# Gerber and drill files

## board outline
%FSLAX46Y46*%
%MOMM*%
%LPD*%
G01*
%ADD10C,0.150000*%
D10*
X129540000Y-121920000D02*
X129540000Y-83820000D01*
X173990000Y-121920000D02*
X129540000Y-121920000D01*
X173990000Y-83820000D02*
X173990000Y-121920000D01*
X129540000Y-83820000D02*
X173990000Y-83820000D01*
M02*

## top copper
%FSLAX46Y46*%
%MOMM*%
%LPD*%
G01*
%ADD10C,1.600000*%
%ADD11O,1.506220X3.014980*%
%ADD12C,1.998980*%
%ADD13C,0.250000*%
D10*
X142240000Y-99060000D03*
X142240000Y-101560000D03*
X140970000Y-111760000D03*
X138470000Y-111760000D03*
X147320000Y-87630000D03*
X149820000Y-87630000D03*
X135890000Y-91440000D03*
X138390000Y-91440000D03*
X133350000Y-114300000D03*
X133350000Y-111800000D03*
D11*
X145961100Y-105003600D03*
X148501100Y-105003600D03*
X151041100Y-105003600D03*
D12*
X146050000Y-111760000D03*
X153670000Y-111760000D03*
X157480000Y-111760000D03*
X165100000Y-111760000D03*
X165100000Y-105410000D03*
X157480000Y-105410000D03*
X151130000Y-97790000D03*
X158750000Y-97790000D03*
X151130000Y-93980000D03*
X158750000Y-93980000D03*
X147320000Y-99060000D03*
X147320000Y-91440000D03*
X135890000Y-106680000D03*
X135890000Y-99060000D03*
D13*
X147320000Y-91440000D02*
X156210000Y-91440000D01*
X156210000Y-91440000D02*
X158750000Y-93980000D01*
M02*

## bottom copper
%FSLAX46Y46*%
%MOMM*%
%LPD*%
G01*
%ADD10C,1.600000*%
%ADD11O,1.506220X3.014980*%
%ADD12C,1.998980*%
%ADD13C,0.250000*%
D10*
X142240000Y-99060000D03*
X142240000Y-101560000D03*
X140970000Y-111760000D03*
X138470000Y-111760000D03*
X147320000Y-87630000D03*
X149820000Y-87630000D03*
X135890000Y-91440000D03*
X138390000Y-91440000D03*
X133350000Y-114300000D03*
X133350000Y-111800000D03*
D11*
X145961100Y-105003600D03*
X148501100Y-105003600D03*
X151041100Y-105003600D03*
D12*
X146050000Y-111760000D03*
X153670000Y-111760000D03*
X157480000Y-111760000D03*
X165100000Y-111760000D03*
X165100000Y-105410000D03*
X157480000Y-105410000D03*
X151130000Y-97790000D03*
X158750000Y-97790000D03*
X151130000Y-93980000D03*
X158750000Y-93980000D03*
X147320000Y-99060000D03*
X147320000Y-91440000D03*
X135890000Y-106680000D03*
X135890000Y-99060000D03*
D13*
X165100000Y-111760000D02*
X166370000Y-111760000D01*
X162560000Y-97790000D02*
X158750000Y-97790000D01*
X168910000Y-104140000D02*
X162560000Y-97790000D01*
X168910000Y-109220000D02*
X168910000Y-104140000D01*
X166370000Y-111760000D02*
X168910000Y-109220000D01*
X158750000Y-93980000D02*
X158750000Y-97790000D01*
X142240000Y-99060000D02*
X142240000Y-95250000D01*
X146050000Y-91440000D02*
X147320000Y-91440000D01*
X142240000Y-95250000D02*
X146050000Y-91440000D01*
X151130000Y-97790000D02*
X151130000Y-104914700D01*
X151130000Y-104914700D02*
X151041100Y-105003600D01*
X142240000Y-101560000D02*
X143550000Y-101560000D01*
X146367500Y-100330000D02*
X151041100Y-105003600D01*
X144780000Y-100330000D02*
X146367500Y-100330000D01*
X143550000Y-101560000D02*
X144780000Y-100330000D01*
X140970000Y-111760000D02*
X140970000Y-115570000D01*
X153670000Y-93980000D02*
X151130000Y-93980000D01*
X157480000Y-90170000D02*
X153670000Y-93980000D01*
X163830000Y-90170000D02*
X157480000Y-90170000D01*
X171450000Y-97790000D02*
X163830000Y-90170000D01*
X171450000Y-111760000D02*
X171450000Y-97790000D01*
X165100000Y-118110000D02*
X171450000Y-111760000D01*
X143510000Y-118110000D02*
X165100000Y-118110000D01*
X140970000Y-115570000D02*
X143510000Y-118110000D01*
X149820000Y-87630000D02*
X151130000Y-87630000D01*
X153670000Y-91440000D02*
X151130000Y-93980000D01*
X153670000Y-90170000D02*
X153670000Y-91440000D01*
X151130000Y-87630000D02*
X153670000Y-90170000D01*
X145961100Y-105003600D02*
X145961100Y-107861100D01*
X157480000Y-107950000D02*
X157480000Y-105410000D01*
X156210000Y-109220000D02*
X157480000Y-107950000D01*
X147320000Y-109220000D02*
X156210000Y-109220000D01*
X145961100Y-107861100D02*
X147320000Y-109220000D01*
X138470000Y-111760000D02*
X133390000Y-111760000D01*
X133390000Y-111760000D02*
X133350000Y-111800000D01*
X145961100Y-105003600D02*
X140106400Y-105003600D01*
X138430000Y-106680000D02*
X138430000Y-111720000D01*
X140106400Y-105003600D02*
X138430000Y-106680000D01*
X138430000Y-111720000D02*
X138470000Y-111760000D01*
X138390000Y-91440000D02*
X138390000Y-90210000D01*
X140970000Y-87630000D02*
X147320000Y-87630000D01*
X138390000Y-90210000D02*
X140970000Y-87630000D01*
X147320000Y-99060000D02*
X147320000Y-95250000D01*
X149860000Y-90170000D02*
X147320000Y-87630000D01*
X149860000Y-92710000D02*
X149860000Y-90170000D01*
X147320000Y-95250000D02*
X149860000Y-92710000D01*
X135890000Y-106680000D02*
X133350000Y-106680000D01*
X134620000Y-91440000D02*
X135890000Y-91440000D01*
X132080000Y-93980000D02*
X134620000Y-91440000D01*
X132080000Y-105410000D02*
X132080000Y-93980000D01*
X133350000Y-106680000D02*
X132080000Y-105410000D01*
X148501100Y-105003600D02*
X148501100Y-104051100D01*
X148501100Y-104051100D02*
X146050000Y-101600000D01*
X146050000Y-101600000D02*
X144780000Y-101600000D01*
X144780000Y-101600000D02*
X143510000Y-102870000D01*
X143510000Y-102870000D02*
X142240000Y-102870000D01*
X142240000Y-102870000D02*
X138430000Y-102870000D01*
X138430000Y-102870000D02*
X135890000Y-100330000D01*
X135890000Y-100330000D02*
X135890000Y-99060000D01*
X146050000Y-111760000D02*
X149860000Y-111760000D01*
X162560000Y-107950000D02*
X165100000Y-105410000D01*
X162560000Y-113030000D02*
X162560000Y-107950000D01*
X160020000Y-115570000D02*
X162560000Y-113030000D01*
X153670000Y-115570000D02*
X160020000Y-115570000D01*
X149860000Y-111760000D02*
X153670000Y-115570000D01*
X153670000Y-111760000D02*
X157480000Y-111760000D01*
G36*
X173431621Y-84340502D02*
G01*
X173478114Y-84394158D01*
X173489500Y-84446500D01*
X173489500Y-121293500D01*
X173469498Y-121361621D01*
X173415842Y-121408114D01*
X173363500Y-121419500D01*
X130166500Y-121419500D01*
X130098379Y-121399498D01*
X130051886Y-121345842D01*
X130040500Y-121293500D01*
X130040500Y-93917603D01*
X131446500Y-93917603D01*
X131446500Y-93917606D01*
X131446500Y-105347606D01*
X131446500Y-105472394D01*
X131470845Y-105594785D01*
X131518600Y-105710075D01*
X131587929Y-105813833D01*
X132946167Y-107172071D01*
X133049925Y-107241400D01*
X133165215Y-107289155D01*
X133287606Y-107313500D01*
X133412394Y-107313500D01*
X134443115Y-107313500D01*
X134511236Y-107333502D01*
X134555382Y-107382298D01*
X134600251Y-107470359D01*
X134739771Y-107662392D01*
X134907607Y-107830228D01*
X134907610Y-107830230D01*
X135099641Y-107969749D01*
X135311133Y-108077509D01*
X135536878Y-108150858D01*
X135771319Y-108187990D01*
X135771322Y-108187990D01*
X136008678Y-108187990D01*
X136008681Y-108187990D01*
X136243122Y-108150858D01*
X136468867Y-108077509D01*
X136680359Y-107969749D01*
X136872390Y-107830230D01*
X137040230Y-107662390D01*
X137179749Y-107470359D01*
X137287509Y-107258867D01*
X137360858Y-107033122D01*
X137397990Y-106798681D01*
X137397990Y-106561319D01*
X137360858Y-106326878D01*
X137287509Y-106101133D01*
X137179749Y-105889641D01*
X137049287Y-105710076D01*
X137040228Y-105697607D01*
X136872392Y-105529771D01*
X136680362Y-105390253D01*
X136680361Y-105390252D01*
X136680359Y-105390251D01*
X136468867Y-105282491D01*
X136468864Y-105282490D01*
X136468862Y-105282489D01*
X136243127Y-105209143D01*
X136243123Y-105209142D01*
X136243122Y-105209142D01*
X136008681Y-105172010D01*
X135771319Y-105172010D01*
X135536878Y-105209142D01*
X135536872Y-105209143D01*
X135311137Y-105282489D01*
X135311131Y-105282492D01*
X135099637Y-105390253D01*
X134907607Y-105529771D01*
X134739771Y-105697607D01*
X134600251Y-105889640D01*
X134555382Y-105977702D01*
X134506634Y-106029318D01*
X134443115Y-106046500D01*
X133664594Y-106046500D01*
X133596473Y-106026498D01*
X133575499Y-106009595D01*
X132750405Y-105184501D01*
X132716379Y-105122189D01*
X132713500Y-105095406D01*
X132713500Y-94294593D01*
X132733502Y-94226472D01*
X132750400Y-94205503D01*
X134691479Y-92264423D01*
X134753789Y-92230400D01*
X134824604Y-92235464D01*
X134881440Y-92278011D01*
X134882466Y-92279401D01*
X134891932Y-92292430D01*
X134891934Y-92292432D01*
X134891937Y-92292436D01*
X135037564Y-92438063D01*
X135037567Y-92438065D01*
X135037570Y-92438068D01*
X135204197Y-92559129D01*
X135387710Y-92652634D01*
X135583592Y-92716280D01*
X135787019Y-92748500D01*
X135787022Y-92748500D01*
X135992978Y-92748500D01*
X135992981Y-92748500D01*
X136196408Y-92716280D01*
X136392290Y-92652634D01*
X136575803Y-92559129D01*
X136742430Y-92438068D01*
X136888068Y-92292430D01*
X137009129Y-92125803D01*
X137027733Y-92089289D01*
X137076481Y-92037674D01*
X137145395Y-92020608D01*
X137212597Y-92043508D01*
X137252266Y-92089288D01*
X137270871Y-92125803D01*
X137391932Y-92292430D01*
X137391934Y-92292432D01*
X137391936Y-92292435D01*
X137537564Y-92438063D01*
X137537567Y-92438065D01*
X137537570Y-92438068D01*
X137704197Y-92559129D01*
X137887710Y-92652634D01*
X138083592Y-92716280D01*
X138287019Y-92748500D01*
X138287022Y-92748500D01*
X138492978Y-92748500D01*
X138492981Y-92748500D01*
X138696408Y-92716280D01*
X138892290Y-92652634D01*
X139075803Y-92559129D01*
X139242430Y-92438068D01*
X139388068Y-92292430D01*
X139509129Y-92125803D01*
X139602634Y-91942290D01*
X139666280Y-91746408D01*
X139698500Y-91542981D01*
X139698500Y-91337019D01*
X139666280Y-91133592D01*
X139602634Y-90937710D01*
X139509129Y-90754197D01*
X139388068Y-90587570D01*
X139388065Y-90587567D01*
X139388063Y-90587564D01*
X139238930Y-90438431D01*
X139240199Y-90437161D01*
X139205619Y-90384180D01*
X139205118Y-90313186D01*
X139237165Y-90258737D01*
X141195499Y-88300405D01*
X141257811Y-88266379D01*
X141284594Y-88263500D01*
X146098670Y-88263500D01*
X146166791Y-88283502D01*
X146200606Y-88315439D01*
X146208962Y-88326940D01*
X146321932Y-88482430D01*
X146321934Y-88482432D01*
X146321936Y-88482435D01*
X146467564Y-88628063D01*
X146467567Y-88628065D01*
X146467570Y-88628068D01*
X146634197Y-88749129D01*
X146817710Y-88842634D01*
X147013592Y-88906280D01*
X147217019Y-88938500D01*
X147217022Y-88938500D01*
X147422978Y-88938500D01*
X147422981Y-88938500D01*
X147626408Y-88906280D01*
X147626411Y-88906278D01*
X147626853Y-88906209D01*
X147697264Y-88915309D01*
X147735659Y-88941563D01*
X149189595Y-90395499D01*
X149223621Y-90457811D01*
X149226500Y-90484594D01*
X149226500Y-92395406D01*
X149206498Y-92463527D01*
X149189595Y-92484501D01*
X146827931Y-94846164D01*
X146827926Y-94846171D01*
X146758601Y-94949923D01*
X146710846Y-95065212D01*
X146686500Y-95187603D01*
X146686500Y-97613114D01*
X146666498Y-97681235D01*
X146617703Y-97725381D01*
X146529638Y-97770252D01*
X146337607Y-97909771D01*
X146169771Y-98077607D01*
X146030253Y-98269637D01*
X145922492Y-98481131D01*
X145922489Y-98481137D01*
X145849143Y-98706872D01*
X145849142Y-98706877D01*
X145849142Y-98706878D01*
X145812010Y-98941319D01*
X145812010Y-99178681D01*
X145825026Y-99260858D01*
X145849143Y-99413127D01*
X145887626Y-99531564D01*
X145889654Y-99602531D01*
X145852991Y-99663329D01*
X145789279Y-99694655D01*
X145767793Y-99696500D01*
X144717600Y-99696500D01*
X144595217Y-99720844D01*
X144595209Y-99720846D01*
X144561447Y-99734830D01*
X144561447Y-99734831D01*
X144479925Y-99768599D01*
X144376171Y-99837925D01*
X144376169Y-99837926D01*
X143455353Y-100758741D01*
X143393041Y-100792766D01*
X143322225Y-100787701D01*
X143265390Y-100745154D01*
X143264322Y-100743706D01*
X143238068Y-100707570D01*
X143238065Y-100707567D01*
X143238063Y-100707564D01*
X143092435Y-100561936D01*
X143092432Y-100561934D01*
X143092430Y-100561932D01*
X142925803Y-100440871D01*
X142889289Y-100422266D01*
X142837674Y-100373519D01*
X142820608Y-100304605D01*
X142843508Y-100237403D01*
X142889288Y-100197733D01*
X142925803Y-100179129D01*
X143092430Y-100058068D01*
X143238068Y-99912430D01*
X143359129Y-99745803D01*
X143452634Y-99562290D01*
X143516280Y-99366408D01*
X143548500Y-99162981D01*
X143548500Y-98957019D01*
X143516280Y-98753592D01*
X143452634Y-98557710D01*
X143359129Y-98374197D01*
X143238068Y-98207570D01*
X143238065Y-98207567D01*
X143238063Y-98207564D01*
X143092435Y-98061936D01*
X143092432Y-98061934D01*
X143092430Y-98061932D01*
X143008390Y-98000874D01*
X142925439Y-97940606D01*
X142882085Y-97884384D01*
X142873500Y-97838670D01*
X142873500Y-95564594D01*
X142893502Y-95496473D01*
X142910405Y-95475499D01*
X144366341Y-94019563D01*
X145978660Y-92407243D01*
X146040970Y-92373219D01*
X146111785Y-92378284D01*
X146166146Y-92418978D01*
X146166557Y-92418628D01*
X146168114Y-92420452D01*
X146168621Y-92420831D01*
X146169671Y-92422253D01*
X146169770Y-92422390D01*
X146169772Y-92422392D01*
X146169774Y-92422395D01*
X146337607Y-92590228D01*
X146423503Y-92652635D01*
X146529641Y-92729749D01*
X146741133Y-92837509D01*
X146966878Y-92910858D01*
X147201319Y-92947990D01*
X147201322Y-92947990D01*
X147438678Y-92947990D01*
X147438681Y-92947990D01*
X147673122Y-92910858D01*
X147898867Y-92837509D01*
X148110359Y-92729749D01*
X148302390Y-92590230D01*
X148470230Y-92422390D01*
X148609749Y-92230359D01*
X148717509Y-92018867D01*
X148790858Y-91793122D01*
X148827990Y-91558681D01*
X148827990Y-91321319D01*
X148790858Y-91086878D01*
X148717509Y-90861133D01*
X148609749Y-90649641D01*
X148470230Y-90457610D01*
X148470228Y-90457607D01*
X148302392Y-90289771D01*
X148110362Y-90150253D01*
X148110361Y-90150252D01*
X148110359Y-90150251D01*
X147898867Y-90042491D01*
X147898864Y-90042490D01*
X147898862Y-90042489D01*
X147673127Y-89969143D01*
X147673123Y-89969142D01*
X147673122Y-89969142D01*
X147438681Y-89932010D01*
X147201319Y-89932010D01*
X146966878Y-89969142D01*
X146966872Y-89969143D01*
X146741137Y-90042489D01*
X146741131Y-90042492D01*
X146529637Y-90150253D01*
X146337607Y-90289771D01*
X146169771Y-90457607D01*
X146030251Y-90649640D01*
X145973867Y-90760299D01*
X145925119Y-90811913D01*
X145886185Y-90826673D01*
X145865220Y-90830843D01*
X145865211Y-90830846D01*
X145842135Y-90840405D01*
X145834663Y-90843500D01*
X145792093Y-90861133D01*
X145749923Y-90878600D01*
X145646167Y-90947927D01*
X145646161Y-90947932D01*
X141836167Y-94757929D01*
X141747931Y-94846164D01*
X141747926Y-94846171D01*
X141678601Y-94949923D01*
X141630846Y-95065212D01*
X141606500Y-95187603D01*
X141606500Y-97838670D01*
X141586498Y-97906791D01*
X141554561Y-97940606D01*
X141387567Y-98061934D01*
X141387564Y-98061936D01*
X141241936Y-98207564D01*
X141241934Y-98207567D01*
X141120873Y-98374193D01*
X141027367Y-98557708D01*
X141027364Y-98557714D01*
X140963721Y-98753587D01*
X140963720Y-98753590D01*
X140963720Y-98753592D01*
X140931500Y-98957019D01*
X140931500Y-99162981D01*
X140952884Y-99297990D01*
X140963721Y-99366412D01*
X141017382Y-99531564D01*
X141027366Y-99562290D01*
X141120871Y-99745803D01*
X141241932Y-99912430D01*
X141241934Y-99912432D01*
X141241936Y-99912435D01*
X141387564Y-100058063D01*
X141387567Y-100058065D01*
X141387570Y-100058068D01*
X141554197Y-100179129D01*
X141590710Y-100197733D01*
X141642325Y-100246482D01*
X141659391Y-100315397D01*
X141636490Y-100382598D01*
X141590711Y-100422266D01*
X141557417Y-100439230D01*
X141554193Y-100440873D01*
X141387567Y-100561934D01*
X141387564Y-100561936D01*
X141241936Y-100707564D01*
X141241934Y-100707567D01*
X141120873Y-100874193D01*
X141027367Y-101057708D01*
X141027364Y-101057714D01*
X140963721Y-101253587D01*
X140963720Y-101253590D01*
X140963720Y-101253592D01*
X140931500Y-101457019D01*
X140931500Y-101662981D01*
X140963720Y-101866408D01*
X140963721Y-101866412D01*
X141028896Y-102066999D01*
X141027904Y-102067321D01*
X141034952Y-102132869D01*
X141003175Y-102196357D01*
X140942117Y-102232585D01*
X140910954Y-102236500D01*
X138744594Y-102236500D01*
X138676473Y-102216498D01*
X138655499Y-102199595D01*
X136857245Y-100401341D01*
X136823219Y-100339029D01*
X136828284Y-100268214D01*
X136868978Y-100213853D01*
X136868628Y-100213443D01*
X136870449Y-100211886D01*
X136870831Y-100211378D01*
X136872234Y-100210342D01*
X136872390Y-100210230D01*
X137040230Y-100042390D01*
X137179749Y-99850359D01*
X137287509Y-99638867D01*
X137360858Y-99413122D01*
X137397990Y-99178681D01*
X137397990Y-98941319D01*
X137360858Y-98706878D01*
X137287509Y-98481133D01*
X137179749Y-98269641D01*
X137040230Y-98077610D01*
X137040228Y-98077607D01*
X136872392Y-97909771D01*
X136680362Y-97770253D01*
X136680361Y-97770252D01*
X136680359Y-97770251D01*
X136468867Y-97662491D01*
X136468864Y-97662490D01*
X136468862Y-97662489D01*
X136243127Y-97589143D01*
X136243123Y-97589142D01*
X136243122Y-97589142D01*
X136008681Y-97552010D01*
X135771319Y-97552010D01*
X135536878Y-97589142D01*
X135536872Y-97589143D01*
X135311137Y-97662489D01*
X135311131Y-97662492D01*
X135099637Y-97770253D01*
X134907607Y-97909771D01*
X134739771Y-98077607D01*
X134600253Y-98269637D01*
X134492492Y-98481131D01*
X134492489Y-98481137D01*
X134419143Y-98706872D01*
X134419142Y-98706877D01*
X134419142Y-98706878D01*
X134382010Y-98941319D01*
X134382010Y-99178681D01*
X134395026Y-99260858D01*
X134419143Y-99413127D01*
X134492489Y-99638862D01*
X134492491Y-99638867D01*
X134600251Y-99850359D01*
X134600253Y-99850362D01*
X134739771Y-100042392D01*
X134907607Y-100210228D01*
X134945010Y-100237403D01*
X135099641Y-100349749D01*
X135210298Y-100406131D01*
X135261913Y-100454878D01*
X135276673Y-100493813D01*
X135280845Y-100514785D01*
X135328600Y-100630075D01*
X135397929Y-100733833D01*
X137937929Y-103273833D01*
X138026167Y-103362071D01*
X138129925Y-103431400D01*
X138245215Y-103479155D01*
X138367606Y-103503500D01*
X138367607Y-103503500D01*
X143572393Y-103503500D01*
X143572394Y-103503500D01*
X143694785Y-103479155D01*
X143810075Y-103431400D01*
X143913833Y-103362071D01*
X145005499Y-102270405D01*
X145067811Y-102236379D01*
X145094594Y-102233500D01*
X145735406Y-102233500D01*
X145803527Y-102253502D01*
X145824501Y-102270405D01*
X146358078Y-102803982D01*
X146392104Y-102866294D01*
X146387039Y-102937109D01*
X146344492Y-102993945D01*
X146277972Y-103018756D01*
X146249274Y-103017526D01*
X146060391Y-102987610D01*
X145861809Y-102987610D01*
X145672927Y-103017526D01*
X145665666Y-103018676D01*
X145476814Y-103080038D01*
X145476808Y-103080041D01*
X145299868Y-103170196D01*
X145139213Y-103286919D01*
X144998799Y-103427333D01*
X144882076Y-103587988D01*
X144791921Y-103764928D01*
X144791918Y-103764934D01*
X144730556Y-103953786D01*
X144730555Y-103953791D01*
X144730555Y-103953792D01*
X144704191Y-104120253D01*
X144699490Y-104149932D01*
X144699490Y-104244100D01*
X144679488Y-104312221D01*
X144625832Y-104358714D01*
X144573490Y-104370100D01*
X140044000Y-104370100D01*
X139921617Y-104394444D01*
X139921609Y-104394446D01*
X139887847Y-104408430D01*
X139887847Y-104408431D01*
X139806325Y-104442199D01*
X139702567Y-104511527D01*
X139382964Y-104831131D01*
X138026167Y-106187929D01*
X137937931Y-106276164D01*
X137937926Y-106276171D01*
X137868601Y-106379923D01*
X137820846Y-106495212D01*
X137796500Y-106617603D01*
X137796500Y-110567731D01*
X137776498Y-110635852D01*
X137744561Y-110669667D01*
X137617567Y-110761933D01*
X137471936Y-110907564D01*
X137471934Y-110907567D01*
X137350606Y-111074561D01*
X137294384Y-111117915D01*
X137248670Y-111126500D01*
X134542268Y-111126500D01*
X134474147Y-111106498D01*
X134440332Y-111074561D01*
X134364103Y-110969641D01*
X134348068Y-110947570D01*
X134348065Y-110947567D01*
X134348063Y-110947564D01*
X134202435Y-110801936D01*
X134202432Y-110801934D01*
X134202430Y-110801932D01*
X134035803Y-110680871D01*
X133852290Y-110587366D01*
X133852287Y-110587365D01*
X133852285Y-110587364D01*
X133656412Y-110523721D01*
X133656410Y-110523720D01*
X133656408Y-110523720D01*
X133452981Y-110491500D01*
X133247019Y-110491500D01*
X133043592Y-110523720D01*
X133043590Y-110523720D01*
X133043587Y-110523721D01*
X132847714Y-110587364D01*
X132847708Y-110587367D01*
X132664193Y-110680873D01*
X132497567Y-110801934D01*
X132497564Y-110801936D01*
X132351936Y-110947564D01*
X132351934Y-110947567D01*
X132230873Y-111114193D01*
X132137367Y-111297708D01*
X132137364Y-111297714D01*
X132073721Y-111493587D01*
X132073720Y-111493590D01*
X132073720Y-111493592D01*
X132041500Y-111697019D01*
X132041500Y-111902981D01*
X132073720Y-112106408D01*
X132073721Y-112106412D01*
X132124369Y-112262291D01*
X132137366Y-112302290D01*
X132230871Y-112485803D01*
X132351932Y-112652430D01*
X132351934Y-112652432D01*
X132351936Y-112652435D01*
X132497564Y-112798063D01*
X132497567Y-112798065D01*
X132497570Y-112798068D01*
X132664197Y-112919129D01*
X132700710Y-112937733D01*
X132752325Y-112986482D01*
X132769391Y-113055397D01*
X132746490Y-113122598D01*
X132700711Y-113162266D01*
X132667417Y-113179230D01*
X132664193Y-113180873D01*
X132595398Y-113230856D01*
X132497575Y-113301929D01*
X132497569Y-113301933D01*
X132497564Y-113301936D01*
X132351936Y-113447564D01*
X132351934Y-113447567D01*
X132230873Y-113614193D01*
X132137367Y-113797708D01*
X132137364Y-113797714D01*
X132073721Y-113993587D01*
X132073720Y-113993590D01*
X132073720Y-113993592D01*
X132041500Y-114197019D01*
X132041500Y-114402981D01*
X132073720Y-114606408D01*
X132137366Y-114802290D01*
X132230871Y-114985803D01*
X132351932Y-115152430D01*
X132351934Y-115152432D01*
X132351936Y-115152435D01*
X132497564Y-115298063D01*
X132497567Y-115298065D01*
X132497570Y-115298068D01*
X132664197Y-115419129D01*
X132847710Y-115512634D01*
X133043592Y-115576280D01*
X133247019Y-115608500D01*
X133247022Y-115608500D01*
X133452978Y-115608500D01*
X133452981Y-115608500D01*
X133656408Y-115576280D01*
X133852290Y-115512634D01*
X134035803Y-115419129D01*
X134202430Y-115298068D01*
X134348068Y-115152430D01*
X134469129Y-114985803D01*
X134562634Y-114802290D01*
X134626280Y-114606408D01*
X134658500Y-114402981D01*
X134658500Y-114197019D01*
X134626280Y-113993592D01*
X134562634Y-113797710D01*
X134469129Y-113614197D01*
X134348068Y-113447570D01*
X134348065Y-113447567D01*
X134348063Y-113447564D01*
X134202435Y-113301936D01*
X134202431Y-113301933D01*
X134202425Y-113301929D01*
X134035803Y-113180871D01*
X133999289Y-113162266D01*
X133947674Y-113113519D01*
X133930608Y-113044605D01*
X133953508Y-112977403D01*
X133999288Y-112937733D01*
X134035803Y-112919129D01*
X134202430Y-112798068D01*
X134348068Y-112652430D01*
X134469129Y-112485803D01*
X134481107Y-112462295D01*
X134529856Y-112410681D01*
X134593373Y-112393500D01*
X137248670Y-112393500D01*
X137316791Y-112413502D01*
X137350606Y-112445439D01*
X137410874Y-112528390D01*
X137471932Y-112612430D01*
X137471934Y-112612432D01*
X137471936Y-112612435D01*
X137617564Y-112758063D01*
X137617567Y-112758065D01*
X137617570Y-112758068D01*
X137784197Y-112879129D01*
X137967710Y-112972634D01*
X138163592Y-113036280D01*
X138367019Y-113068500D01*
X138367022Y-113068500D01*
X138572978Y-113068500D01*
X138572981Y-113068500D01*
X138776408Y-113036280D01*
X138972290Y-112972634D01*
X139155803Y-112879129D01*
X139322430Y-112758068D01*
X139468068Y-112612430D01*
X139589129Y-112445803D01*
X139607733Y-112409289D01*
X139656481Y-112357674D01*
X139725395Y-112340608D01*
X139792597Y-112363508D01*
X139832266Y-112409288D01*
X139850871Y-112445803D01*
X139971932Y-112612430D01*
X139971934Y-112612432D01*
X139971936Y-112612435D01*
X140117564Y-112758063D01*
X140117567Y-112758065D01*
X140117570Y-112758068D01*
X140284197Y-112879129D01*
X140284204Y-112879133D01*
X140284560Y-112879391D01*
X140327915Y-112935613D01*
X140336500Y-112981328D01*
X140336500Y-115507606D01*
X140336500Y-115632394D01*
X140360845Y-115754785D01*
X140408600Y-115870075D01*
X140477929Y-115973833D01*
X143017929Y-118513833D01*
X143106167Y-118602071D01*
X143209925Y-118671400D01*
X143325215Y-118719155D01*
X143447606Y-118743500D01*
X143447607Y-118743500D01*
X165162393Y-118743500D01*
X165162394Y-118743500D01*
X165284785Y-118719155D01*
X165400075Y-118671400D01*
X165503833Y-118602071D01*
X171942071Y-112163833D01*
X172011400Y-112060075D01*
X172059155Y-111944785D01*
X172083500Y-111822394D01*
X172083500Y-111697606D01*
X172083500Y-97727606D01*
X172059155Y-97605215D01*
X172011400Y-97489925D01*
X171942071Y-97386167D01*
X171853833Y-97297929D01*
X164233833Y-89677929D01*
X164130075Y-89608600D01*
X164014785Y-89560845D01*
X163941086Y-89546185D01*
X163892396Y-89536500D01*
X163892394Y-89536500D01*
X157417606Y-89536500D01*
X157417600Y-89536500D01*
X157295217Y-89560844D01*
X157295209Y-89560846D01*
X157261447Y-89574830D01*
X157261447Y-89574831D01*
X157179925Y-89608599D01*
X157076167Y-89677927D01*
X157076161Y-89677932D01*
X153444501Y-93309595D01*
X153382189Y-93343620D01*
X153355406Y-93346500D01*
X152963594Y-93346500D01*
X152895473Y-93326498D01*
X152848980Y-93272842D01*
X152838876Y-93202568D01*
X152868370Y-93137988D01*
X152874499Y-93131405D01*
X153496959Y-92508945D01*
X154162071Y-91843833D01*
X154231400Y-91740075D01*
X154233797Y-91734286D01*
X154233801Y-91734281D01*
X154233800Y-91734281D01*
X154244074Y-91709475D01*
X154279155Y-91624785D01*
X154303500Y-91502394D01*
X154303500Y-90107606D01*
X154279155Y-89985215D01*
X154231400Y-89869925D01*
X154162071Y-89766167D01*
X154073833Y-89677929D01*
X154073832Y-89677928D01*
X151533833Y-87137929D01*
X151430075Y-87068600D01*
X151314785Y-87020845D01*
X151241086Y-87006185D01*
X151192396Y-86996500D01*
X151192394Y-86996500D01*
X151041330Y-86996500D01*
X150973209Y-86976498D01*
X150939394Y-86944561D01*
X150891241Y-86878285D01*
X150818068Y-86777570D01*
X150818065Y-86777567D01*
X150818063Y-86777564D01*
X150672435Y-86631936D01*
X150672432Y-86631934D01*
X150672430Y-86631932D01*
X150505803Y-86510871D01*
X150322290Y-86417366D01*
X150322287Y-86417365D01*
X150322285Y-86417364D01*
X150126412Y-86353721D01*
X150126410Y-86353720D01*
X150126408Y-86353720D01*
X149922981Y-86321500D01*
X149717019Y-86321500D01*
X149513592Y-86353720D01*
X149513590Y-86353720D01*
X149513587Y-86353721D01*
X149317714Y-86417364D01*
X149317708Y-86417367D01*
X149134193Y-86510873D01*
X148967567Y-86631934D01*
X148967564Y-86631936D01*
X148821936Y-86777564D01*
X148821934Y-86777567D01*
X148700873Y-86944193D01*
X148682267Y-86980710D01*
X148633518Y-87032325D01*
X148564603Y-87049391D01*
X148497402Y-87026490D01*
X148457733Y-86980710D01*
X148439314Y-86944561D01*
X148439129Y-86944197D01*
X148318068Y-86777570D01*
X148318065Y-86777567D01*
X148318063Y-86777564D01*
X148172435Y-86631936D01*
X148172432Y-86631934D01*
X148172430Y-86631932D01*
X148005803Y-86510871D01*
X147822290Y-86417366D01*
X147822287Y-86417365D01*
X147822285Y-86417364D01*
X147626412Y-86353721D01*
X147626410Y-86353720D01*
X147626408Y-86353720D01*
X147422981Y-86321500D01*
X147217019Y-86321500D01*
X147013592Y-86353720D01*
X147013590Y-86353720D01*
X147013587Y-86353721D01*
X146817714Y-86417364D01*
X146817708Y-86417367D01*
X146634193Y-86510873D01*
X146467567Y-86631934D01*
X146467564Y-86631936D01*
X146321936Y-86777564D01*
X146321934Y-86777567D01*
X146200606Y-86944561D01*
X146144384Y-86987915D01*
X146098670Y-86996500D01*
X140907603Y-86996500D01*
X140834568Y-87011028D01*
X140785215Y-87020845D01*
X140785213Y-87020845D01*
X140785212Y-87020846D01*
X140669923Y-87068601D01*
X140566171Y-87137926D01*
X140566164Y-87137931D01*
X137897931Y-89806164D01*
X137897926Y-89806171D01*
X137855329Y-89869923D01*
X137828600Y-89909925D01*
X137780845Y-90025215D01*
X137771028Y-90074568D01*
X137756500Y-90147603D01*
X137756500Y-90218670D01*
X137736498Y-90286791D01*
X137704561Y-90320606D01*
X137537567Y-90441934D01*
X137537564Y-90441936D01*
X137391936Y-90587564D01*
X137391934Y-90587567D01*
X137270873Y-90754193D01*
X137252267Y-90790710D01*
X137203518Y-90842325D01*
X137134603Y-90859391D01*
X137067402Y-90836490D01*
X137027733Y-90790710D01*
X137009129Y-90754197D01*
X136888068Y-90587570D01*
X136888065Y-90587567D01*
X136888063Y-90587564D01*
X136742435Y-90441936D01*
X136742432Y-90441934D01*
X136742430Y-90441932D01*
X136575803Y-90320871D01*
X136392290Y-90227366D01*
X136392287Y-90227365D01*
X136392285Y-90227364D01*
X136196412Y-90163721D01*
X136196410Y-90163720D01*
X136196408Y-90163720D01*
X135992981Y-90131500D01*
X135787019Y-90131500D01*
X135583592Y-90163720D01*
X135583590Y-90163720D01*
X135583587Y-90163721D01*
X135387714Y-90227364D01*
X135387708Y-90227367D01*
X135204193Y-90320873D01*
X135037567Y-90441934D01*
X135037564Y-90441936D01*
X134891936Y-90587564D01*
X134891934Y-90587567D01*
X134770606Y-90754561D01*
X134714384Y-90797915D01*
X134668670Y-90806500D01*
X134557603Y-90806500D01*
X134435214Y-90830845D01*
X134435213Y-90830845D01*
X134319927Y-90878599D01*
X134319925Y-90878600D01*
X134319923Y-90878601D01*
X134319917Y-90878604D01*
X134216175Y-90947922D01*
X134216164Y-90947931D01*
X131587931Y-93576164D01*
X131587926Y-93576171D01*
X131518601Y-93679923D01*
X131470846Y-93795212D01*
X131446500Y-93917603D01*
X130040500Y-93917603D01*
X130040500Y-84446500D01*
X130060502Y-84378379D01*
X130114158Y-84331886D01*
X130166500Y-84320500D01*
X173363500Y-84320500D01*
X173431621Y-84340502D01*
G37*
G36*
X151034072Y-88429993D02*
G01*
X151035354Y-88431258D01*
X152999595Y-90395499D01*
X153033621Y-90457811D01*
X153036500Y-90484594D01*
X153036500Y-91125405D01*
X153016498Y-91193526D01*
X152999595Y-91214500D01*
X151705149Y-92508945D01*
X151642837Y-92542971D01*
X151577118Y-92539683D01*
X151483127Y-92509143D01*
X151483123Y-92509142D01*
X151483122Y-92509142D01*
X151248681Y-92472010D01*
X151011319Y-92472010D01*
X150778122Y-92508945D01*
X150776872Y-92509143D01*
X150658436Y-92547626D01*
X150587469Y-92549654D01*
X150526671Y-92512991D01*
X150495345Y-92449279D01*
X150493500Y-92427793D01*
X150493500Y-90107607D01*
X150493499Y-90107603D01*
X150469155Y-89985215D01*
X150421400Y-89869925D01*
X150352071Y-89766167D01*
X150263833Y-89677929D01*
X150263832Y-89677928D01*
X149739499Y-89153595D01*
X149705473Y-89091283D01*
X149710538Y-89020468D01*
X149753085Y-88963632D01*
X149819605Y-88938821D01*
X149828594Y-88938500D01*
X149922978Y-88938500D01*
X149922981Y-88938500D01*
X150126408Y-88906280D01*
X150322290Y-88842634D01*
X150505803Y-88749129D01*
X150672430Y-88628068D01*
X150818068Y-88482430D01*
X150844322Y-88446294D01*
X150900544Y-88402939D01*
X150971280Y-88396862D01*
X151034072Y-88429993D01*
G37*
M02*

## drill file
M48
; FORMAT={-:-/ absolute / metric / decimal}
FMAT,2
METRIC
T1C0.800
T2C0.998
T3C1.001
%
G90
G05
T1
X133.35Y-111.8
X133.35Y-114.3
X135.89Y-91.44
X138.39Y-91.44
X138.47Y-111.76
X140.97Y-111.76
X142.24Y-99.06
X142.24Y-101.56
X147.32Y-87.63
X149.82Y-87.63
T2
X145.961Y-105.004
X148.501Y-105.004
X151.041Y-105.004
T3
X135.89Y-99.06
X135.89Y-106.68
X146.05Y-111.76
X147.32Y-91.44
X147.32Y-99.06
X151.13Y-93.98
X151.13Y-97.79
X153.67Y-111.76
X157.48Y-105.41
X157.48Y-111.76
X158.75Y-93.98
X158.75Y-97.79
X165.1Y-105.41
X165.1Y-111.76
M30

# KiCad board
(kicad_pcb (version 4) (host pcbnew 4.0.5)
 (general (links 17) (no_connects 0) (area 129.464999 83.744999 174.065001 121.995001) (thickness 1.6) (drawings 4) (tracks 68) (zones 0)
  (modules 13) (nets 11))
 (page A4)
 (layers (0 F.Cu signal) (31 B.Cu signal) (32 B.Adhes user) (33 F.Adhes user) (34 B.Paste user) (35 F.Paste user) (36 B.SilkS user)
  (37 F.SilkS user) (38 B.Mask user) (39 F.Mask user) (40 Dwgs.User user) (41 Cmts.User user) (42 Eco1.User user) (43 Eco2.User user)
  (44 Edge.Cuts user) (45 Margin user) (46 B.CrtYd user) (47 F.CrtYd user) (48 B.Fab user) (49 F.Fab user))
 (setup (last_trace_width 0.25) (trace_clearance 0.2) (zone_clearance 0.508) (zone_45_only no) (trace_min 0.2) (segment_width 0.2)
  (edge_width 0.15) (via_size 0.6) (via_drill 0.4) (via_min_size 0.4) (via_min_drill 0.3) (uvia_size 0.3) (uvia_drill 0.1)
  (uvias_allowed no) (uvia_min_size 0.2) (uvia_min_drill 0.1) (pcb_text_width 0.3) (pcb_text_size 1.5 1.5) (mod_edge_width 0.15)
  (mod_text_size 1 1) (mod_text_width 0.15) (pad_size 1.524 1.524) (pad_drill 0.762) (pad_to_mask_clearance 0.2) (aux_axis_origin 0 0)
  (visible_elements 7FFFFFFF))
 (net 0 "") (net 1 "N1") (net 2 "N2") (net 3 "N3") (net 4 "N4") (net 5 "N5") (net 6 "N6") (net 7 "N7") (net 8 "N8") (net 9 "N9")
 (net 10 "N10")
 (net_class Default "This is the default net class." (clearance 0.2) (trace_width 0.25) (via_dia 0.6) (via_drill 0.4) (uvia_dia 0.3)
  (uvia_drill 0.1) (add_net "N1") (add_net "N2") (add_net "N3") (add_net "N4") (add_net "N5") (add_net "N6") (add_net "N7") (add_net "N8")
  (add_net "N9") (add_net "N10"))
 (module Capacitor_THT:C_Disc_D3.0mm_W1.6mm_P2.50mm (layer F.Cu) (at 142.24 99.06 270)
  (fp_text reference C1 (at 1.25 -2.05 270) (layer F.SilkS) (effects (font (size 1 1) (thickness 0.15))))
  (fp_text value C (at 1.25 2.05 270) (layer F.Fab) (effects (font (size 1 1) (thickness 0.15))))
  (pad 1 thru_hole circle (at 0 0 270) (size 1.6 1.6) (drill 0.8) (layers *.Cu *.Mask) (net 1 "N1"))
  (pad 2 thru_hole circle (at 2.5 0 270) (size 1.6 1.6) (drill 0.8) (layers *.Cu *.Mask) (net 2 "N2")))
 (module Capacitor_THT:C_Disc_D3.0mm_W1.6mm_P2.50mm (layer F.Cu) (at 140.97 111.76 180)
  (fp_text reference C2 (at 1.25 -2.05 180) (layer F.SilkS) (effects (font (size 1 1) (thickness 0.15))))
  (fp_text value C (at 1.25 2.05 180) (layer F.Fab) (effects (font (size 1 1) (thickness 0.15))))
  (pad 1 thru_hole circle (at 0 0 180) (size 1.6 1.6) (drill 0.8) (layers *.Cu *.Mask) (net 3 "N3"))
  (pad 2 thru_hole circle (at 2.5 0 180) (size 1.6 1.6) (drill 0.8) (layers *.Cu *.Mask) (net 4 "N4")))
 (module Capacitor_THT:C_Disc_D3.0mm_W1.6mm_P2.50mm (layer F.Cu) (at 147.32 87.63)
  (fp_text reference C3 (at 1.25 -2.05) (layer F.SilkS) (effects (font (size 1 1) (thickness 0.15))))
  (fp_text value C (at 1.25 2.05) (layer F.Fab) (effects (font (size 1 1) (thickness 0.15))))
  (pad 1 thru_hole circle (at 0 0) (size 1.6 1.6) (drill 0.8) (layers *.Cu *.Mask) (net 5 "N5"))
  (pad 2 thru_hole circle (at 2.5 0) (size 1.6 1.6) (drill 0.8) (layers *.Cu *.Mask) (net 3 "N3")))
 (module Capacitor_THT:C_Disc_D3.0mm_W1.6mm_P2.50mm (layer F.Cu) (at 135.89 91.44)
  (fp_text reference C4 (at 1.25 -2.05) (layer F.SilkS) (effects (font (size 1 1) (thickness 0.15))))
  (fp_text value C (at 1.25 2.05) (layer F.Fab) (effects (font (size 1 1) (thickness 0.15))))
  (pad 1 thru_hole circle (at 0 0) (size 1.6 1.6) (drill 0.8) (layers *.Cu *.Mask) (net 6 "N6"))
  (pad 2 thru_hole circle (at 2.5 0) (size 1.6 1.6) (drill 0.8) (layers *.Cu *.Mask) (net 5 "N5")))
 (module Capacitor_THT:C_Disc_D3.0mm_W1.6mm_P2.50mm (layer F.Cu) (at 133.35 114.3 90)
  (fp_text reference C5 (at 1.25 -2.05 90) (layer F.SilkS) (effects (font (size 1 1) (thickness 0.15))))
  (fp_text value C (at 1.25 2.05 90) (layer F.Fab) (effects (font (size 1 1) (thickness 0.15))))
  (pad 1 thru_hole circle (at 0 0 90) (size 1.6 1.6) (drill 0.8) (layers *.Cu *.Mask) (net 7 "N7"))
  (pad 2 thru_hole circle (at 2.5 0 90) (size 1.6 1.6) (drill 0.8) (layers *.Cu *.Mask) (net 4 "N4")))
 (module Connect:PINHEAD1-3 (layer F.Cu) (at 148.5011 105.0036)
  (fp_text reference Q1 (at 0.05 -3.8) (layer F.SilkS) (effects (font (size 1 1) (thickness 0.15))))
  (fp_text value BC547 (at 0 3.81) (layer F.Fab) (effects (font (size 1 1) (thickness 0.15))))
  (pad 1 thru_hole oval (at -2.54 0) (size 1.50622 3.01498) (drill 0.99822) (layers *.Cu *.Mask) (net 4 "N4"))
  (pad 2 thru_hole oval (at 0 0) (size 1.50622 3.01498) (drill 0.99822) (layers *.Cu *.Mask) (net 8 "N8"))
  (pad 3 thru_hole oval (at 2.54 0) (size 1.50622 3.01498) (drill 0.99822) (layers *.Cu *.Mask) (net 2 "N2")))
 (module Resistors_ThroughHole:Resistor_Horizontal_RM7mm (layer F.Cu) (at 146.05 111.76)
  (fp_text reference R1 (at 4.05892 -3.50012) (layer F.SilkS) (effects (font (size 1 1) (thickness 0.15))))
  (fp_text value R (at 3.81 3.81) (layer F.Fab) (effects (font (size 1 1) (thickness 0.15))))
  (pad 1 thru_hole circle (at 0 0) (size 1.99898 1.99898) (drill 1.00076) (layers *.Cu *.SilkS *.Mask) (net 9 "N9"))
  (pad 2 thru_hole circle (at 7.62 0) (size 1.99898 1.99898) (drill 1.00076) (layers *.Cu *.SilkS *.Mask) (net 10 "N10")))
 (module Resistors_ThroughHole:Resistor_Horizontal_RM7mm (layer F.Cu) (at 157.48 111.76)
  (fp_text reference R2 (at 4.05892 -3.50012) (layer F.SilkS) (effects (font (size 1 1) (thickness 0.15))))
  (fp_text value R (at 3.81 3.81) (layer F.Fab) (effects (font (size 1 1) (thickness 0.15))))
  (pad 1 thru_hole circle (at 0 0) (size 1.99898 1.99898) (drill 1.00076) (layers *.Cu *.SilkS *.Mask) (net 10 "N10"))
  (pad 2 thru_hole circle (at 7.62 0) (size 1.99898 1.99898) (drill 1.00076) (layers *.Cu *.SilkS *.Mask) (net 1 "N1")))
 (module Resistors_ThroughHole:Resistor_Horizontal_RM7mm (layer F.Cu) (at 165.1 105.41 180)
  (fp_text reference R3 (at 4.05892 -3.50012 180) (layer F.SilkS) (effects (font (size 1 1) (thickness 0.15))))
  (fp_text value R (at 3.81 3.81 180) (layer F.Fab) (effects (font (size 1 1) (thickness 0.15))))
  (pad 1 thru_hole circle (at 0 0 180) (size 1.99898 1.99898) (drill 1.00076) (layers *.Cu *.SilkS *.Mask) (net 9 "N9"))
  (pad 2 thru_hole circle (at 7.62 0 180) (size 1.99898 1.99898) (drill 1.00076) (layers *.Cu *.SilkS *.Mask) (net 4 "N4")))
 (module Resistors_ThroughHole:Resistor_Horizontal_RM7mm (layer F.Cu) (at 151.13 97.79)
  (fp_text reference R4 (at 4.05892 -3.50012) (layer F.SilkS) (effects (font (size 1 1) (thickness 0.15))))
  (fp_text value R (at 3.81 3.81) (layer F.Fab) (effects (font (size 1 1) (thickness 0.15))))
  (pad 1 thru_hole circle (at 0 0) (size 1.99898 1.99898) (drill 1.00076) (layers *.Cu *.SilkS *.Mask) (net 2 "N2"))
  (pad 2 thru_hole circle (at 7.62 0) (size 1.99898 1.99898) (drill 1.00076) (layers *.Cu *.SilkS *.Mask) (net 1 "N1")))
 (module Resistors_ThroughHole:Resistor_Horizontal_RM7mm (layer F.Cu) (at 151.13 93.98)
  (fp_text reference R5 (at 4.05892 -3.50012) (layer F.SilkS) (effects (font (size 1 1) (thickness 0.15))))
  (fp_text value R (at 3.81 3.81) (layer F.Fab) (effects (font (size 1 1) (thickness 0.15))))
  (pad 1 thru_hole circle (at 0 0) (size 1.99898 1.99898) (drill 1.00076) (layers *.Cu *.SilkS *.Mask) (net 3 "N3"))
  (pad 2 thru_hole circle (at 7.62 0) (size 1.99898 1.99898) (drill 1.00076) (layers *.Cu *.SilkS *.Mask) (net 1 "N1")))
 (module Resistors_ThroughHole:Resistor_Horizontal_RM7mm (layer F.Cu) (at 147.32 99.06 90)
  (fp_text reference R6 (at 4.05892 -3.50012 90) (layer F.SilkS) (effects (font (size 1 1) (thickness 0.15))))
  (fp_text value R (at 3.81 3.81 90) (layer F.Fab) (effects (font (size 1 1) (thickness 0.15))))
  (pad 1 thru_hole circle (at 0 0 90) (size 1.99898 1.99898) (drill 1.00076) (layers *.Cu *.SilkS *.Mask) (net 5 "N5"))
  (pad 2 thru_hole circle (at 7.62 0 90) (size 1.99898 1.99898) (drill 1.00076) (layers *.Cu *.SilkS *.Mask) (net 1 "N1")))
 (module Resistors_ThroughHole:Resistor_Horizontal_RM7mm (layer F.Cu) (at 135.89 106.68 90)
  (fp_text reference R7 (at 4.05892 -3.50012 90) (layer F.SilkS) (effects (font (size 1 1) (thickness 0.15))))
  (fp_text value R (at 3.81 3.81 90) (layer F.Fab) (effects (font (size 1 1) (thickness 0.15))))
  (pad 1 thru_hole circle (at 0 0 90) (size 1.99898 1.99898) (drill 1.00076) (layers *.Cu *.SilkS *.Mask) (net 6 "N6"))
  (pad 2 thru_hole circle (at 7.62 0 90) (size 1.99898 1.99898) (drill 1.00076) (layers *.Cu *.SilkS *.Mask) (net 8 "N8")))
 (gr_line (start 129.54 121.92) (end 129.54 83.82) (angle 90) (layer Edge.Cuts) (width 0.15))
 (gr_line (start 173.99 121.92) (end 129.54 121.92) (angle 90) (layer Edge.Cuts) (width 0.15))
 (gr_line (start 173.99 83.82) (end 173.99 121.92) (angle 90) (layer Edge.Cuts) (width 0.15))
 (gr_line (start 129.54 83.82) (end 173.99 83.82) (angle 90) (layer Edge.Cuts) (width 0.15))
 (segment (start 147.32 91.44) (end 156.21 91.44) (width 0.25) (layer F.Cu) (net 1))
 (segment (start 156.21 91.44) (end 158.75 93.98) (width 0.25) (layer F.Cu) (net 1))
 (segment (start 165.1 111.76) (end 166.37 111.76) (width 0.25) (layer B.Cu) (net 1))
 (segment (start 162.56 97.79) (end 158.75 97.79) (width 0.25) (layer B.Cu) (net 1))
 (segment (start 168.91 104.14) (end 162.56 97.79) (width 0.25) (layer B.Cu) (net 1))
 (segment (start 168.91 109.22) (end 168.91 104.14) (width 0.25) (layer B.Cu) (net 1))
 (segment (start 166.37 111.76) (end 168.91 109.22) (width 0.25) (layer B.Cu) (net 1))
 (segment (start 158.75 93.98) (end 158.75 97.79) (width 0.25) (layer B.Cu) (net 1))
 (segment (start 142.24 99.06) (end 142.24 95.25) (width 0.25) (layer B.Cu) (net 1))
 (segment (start 146.05 91.44) (end 147.32 91.44) (width 0.25) (layer B.Cu) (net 1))
 (segment (start 142.24 95.25) (end 146.05 91.44) (width 0.25) (layer B.Cu) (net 1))
 (segment (start 151.13 97.79) (end 151.13 104.9147) (width 0.25) (layer B.Cu) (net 2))
 (segment (start 151.13 104.9147) (end 151.0411 105.0036) (width 0.25) (layer B.Cu) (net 2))
 (segment (start 142.24 101.56) (end 143.55 101.56) (width 0.25) (layer B.Cu) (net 2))
 (segment (start 146.3675 100.33) (end 151.0411 105.0036) (width 0.25) (layer B.Cu) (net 2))
 (segment (start 144.78 100.33) (end 146.3675 100.33) (width 0.25) (layer B.Cu) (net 2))
 (segment (start 143.55 101.56) (end 144.78 100.33) (width 0.25) (layer B.Cu) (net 2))
 (segment (start 140.97 111.76) (end 140.97 115.57) (width 0.25) (layer B.Cu) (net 3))
 (segment (start 153.67 93.98) (end 151.13 93.98) (width 0.25) (layer B.Cu) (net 3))
 (segment (start 157.48 90.17) (end 153.67 93.98) (width 0.25) (layer B.Cu) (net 3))
 (segment (start 163.83 90.17) (end 157.48 90.17) (width 0.25) (layer B.Cu) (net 3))
 (segment (start 171.45 97.79) (end 163.83 90.17) (width 0.25) (layer B.Cu) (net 3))
 (segment (start 171.45 111.76) (end 171.45 97.79) (width 0.25) (layer B.Cu) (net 3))
 (segment (start 165.1 118.11) (end 171.45 111.76) (width 0.25) (layer B.Cu) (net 3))
 (segment (start 143.51 118.11) (end 165.1 118.11) (width 0.25) (layer B.Cu) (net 3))
 (segment (start 140.97 115.57) (end 143.51 118.11) (width 0.25) (layer B.Cu) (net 3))
 (segment (start 149.82 87.63) (end 151.13 87.63) (width 0.25) (layer B.Cu) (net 3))
 (segment (start 153.67 91.44) (end 151.13 93.98) (width 0.25) (layer B.Cu) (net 3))
 (segment (start 153.67 90.17) (end 153.67 91.44) (width 0.25) (layer B.Cu) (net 3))
 (segment (start 151.13 87.63) (end 153.67 90.17) (width 0.25) (layer B.Cu) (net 3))
 (segment (start 145.9611 105.0036) (end 145.9611 107.8611) (width 0.25) (layer B.Cu) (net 4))
 (segment (start 157.48 107.95) (end 157.48 105.41) (width 0.25) (layer B.Cu) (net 4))
 (segment (start 156.21 109.22) (end 157.48 107.95) (width 0.25) (layer B.Cu) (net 4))
 (segment (start 147.32 109.22) (end 156.21 109.22) (width 0.25) (layer B.Cu) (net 4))
 (segment (start 145.9611 107.8611) (end 147.32 109.22) (width 0.25) (layer B.Cu) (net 4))
 (segment (start 138.47 111.76) (end 133.39 111.76) (width 0.25) (layer B.Cu) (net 4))
 (segment (start 133.39 111.76) (end 133.35 111.8) (width 0.25) (layer B.Cu) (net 4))
 (segment (start 145.9611 105.0036) (end 140.1064 105.0036) (width 0.25) (layer B.Cu) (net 4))
 (segment (start 138.43 106.68) (end 138.43 111.72) (width 0.25) (layer B.Cu) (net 4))
 (segment (start 140.1064 105.0036) (end 138.43 106.68) (width 0.25) (layer B.Cu) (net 4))
 (segment (start 138.43 111.72) (end 138.47 111.76) (width 0.25) (layer B.Cu) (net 4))
 (segment (start 138.39 91.44) (end 138.39 90.21) (width 0.25) (layer B.Cu) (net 5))
 (segment (start 140.97 87.63) (end 147.32 87.63) (width 0.25) (layer B.Cu) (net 5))
 (segment (start 138.39 90.21) (end 140.97 87.63) (width 0.25) (layer B.Cu) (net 5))
 (segment (start 147.32 99.06) (end 147.32 95.25) (width 0.25) (layer B.Cu) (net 5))
 (segment (start 149.86 90.17) (end 147.32 87.63) (width 0.25) (layer B.Cu) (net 5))
 (segment (start 149.86 92.71) (end 149.86 90.17) (width 0.25) (layer B.Cu) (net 5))
 (segment (start 147.32 95.25) (end 149.86 92.71) (width 0.25) (layer B.Cu) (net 5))
 (segment (start 135.89 106.68) (end 133.35 106.68) (width 0.25) (layer B.Cu) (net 6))
 (segment (start 134.62 91.44) (end 135.89 91.44) (width 0.25) (layer B.Cu) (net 6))
 (segment (start 132.08 93.98) (end 134.62 91.44) (width 0.25) (layer B.Cu) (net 6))
 (segment (start 132.08 105.41) (end 132.08 93.98) (width 0.25) (layer B.Cu) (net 6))
 (segment (start 133.35 106.68) (end 132.08 105.41) (width 0.25) (layer B.Cu) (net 6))
 (segment (start 148.5011 105.0036) (end 148.5011 104.0511) (width 0.25) (layer B.Cu) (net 8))
 (segment (start 148.5011 104.0511) (end 146.05 101.6) (width 0.25) (layer B.Cu) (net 8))
 (segment (start 146.05 101.6) (end 144.78 101.6) (width 0.25) (layer B.Cu) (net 8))
 (segment (start 144.78 101.6) (end 143.51 102.87) (width 0.25) (layer B.Cu) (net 8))
 (segment (start 143.51 102.87) (end 142.24 102.87) (width 0.25) (layer B.Cu) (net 8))
 (segment (start 142.24 102.87) (end 138.43 102.87) (width 0.25) (layer B.Cu) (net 8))
 (segment (start 138.43 102.87) (end 135.89 100.33) (width 0.25) (layer B.Cu) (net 8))
 (segment (start 135.89 100.33) (end 135.89 99.06) (width 0.25) (layer B.Cu) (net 8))
 (segment (start 146.05 111.76) (end 149.86 111.76) (width 0.25) (layer B.Cu) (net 9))
 (segment (start 162.56 107.95) (end 165.1 105.41) (width 0.25) (layer B.Cu) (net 9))
 (segment (start 162.56 113.03) (end 162.56 107.95) (width 0.25) (layer B.Cu) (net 9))
 (segment (start 160.02 115.57) (end 162.56 113.03) (width 0.25) (layer B.Cu) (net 9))
 (segment (start 153.67 115.57) (end 160.02 115.57) (width 0.25) (layer B.Cu) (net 9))
 (segment (start 149.86 111.76) (end 153.67 115.57) (width 0.25) (layer B.Cu) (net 9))
 (segment (start 153.67 111.76) (end 157.48 111.76) (width 0.25) (layer B.Cu) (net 10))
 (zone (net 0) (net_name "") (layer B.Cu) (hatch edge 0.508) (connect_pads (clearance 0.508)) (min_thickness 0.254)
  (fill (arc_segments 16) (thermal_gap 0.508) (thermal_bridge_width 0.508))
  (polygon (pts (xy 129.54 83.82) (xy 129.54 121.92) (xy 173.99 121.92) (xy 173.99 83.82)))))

